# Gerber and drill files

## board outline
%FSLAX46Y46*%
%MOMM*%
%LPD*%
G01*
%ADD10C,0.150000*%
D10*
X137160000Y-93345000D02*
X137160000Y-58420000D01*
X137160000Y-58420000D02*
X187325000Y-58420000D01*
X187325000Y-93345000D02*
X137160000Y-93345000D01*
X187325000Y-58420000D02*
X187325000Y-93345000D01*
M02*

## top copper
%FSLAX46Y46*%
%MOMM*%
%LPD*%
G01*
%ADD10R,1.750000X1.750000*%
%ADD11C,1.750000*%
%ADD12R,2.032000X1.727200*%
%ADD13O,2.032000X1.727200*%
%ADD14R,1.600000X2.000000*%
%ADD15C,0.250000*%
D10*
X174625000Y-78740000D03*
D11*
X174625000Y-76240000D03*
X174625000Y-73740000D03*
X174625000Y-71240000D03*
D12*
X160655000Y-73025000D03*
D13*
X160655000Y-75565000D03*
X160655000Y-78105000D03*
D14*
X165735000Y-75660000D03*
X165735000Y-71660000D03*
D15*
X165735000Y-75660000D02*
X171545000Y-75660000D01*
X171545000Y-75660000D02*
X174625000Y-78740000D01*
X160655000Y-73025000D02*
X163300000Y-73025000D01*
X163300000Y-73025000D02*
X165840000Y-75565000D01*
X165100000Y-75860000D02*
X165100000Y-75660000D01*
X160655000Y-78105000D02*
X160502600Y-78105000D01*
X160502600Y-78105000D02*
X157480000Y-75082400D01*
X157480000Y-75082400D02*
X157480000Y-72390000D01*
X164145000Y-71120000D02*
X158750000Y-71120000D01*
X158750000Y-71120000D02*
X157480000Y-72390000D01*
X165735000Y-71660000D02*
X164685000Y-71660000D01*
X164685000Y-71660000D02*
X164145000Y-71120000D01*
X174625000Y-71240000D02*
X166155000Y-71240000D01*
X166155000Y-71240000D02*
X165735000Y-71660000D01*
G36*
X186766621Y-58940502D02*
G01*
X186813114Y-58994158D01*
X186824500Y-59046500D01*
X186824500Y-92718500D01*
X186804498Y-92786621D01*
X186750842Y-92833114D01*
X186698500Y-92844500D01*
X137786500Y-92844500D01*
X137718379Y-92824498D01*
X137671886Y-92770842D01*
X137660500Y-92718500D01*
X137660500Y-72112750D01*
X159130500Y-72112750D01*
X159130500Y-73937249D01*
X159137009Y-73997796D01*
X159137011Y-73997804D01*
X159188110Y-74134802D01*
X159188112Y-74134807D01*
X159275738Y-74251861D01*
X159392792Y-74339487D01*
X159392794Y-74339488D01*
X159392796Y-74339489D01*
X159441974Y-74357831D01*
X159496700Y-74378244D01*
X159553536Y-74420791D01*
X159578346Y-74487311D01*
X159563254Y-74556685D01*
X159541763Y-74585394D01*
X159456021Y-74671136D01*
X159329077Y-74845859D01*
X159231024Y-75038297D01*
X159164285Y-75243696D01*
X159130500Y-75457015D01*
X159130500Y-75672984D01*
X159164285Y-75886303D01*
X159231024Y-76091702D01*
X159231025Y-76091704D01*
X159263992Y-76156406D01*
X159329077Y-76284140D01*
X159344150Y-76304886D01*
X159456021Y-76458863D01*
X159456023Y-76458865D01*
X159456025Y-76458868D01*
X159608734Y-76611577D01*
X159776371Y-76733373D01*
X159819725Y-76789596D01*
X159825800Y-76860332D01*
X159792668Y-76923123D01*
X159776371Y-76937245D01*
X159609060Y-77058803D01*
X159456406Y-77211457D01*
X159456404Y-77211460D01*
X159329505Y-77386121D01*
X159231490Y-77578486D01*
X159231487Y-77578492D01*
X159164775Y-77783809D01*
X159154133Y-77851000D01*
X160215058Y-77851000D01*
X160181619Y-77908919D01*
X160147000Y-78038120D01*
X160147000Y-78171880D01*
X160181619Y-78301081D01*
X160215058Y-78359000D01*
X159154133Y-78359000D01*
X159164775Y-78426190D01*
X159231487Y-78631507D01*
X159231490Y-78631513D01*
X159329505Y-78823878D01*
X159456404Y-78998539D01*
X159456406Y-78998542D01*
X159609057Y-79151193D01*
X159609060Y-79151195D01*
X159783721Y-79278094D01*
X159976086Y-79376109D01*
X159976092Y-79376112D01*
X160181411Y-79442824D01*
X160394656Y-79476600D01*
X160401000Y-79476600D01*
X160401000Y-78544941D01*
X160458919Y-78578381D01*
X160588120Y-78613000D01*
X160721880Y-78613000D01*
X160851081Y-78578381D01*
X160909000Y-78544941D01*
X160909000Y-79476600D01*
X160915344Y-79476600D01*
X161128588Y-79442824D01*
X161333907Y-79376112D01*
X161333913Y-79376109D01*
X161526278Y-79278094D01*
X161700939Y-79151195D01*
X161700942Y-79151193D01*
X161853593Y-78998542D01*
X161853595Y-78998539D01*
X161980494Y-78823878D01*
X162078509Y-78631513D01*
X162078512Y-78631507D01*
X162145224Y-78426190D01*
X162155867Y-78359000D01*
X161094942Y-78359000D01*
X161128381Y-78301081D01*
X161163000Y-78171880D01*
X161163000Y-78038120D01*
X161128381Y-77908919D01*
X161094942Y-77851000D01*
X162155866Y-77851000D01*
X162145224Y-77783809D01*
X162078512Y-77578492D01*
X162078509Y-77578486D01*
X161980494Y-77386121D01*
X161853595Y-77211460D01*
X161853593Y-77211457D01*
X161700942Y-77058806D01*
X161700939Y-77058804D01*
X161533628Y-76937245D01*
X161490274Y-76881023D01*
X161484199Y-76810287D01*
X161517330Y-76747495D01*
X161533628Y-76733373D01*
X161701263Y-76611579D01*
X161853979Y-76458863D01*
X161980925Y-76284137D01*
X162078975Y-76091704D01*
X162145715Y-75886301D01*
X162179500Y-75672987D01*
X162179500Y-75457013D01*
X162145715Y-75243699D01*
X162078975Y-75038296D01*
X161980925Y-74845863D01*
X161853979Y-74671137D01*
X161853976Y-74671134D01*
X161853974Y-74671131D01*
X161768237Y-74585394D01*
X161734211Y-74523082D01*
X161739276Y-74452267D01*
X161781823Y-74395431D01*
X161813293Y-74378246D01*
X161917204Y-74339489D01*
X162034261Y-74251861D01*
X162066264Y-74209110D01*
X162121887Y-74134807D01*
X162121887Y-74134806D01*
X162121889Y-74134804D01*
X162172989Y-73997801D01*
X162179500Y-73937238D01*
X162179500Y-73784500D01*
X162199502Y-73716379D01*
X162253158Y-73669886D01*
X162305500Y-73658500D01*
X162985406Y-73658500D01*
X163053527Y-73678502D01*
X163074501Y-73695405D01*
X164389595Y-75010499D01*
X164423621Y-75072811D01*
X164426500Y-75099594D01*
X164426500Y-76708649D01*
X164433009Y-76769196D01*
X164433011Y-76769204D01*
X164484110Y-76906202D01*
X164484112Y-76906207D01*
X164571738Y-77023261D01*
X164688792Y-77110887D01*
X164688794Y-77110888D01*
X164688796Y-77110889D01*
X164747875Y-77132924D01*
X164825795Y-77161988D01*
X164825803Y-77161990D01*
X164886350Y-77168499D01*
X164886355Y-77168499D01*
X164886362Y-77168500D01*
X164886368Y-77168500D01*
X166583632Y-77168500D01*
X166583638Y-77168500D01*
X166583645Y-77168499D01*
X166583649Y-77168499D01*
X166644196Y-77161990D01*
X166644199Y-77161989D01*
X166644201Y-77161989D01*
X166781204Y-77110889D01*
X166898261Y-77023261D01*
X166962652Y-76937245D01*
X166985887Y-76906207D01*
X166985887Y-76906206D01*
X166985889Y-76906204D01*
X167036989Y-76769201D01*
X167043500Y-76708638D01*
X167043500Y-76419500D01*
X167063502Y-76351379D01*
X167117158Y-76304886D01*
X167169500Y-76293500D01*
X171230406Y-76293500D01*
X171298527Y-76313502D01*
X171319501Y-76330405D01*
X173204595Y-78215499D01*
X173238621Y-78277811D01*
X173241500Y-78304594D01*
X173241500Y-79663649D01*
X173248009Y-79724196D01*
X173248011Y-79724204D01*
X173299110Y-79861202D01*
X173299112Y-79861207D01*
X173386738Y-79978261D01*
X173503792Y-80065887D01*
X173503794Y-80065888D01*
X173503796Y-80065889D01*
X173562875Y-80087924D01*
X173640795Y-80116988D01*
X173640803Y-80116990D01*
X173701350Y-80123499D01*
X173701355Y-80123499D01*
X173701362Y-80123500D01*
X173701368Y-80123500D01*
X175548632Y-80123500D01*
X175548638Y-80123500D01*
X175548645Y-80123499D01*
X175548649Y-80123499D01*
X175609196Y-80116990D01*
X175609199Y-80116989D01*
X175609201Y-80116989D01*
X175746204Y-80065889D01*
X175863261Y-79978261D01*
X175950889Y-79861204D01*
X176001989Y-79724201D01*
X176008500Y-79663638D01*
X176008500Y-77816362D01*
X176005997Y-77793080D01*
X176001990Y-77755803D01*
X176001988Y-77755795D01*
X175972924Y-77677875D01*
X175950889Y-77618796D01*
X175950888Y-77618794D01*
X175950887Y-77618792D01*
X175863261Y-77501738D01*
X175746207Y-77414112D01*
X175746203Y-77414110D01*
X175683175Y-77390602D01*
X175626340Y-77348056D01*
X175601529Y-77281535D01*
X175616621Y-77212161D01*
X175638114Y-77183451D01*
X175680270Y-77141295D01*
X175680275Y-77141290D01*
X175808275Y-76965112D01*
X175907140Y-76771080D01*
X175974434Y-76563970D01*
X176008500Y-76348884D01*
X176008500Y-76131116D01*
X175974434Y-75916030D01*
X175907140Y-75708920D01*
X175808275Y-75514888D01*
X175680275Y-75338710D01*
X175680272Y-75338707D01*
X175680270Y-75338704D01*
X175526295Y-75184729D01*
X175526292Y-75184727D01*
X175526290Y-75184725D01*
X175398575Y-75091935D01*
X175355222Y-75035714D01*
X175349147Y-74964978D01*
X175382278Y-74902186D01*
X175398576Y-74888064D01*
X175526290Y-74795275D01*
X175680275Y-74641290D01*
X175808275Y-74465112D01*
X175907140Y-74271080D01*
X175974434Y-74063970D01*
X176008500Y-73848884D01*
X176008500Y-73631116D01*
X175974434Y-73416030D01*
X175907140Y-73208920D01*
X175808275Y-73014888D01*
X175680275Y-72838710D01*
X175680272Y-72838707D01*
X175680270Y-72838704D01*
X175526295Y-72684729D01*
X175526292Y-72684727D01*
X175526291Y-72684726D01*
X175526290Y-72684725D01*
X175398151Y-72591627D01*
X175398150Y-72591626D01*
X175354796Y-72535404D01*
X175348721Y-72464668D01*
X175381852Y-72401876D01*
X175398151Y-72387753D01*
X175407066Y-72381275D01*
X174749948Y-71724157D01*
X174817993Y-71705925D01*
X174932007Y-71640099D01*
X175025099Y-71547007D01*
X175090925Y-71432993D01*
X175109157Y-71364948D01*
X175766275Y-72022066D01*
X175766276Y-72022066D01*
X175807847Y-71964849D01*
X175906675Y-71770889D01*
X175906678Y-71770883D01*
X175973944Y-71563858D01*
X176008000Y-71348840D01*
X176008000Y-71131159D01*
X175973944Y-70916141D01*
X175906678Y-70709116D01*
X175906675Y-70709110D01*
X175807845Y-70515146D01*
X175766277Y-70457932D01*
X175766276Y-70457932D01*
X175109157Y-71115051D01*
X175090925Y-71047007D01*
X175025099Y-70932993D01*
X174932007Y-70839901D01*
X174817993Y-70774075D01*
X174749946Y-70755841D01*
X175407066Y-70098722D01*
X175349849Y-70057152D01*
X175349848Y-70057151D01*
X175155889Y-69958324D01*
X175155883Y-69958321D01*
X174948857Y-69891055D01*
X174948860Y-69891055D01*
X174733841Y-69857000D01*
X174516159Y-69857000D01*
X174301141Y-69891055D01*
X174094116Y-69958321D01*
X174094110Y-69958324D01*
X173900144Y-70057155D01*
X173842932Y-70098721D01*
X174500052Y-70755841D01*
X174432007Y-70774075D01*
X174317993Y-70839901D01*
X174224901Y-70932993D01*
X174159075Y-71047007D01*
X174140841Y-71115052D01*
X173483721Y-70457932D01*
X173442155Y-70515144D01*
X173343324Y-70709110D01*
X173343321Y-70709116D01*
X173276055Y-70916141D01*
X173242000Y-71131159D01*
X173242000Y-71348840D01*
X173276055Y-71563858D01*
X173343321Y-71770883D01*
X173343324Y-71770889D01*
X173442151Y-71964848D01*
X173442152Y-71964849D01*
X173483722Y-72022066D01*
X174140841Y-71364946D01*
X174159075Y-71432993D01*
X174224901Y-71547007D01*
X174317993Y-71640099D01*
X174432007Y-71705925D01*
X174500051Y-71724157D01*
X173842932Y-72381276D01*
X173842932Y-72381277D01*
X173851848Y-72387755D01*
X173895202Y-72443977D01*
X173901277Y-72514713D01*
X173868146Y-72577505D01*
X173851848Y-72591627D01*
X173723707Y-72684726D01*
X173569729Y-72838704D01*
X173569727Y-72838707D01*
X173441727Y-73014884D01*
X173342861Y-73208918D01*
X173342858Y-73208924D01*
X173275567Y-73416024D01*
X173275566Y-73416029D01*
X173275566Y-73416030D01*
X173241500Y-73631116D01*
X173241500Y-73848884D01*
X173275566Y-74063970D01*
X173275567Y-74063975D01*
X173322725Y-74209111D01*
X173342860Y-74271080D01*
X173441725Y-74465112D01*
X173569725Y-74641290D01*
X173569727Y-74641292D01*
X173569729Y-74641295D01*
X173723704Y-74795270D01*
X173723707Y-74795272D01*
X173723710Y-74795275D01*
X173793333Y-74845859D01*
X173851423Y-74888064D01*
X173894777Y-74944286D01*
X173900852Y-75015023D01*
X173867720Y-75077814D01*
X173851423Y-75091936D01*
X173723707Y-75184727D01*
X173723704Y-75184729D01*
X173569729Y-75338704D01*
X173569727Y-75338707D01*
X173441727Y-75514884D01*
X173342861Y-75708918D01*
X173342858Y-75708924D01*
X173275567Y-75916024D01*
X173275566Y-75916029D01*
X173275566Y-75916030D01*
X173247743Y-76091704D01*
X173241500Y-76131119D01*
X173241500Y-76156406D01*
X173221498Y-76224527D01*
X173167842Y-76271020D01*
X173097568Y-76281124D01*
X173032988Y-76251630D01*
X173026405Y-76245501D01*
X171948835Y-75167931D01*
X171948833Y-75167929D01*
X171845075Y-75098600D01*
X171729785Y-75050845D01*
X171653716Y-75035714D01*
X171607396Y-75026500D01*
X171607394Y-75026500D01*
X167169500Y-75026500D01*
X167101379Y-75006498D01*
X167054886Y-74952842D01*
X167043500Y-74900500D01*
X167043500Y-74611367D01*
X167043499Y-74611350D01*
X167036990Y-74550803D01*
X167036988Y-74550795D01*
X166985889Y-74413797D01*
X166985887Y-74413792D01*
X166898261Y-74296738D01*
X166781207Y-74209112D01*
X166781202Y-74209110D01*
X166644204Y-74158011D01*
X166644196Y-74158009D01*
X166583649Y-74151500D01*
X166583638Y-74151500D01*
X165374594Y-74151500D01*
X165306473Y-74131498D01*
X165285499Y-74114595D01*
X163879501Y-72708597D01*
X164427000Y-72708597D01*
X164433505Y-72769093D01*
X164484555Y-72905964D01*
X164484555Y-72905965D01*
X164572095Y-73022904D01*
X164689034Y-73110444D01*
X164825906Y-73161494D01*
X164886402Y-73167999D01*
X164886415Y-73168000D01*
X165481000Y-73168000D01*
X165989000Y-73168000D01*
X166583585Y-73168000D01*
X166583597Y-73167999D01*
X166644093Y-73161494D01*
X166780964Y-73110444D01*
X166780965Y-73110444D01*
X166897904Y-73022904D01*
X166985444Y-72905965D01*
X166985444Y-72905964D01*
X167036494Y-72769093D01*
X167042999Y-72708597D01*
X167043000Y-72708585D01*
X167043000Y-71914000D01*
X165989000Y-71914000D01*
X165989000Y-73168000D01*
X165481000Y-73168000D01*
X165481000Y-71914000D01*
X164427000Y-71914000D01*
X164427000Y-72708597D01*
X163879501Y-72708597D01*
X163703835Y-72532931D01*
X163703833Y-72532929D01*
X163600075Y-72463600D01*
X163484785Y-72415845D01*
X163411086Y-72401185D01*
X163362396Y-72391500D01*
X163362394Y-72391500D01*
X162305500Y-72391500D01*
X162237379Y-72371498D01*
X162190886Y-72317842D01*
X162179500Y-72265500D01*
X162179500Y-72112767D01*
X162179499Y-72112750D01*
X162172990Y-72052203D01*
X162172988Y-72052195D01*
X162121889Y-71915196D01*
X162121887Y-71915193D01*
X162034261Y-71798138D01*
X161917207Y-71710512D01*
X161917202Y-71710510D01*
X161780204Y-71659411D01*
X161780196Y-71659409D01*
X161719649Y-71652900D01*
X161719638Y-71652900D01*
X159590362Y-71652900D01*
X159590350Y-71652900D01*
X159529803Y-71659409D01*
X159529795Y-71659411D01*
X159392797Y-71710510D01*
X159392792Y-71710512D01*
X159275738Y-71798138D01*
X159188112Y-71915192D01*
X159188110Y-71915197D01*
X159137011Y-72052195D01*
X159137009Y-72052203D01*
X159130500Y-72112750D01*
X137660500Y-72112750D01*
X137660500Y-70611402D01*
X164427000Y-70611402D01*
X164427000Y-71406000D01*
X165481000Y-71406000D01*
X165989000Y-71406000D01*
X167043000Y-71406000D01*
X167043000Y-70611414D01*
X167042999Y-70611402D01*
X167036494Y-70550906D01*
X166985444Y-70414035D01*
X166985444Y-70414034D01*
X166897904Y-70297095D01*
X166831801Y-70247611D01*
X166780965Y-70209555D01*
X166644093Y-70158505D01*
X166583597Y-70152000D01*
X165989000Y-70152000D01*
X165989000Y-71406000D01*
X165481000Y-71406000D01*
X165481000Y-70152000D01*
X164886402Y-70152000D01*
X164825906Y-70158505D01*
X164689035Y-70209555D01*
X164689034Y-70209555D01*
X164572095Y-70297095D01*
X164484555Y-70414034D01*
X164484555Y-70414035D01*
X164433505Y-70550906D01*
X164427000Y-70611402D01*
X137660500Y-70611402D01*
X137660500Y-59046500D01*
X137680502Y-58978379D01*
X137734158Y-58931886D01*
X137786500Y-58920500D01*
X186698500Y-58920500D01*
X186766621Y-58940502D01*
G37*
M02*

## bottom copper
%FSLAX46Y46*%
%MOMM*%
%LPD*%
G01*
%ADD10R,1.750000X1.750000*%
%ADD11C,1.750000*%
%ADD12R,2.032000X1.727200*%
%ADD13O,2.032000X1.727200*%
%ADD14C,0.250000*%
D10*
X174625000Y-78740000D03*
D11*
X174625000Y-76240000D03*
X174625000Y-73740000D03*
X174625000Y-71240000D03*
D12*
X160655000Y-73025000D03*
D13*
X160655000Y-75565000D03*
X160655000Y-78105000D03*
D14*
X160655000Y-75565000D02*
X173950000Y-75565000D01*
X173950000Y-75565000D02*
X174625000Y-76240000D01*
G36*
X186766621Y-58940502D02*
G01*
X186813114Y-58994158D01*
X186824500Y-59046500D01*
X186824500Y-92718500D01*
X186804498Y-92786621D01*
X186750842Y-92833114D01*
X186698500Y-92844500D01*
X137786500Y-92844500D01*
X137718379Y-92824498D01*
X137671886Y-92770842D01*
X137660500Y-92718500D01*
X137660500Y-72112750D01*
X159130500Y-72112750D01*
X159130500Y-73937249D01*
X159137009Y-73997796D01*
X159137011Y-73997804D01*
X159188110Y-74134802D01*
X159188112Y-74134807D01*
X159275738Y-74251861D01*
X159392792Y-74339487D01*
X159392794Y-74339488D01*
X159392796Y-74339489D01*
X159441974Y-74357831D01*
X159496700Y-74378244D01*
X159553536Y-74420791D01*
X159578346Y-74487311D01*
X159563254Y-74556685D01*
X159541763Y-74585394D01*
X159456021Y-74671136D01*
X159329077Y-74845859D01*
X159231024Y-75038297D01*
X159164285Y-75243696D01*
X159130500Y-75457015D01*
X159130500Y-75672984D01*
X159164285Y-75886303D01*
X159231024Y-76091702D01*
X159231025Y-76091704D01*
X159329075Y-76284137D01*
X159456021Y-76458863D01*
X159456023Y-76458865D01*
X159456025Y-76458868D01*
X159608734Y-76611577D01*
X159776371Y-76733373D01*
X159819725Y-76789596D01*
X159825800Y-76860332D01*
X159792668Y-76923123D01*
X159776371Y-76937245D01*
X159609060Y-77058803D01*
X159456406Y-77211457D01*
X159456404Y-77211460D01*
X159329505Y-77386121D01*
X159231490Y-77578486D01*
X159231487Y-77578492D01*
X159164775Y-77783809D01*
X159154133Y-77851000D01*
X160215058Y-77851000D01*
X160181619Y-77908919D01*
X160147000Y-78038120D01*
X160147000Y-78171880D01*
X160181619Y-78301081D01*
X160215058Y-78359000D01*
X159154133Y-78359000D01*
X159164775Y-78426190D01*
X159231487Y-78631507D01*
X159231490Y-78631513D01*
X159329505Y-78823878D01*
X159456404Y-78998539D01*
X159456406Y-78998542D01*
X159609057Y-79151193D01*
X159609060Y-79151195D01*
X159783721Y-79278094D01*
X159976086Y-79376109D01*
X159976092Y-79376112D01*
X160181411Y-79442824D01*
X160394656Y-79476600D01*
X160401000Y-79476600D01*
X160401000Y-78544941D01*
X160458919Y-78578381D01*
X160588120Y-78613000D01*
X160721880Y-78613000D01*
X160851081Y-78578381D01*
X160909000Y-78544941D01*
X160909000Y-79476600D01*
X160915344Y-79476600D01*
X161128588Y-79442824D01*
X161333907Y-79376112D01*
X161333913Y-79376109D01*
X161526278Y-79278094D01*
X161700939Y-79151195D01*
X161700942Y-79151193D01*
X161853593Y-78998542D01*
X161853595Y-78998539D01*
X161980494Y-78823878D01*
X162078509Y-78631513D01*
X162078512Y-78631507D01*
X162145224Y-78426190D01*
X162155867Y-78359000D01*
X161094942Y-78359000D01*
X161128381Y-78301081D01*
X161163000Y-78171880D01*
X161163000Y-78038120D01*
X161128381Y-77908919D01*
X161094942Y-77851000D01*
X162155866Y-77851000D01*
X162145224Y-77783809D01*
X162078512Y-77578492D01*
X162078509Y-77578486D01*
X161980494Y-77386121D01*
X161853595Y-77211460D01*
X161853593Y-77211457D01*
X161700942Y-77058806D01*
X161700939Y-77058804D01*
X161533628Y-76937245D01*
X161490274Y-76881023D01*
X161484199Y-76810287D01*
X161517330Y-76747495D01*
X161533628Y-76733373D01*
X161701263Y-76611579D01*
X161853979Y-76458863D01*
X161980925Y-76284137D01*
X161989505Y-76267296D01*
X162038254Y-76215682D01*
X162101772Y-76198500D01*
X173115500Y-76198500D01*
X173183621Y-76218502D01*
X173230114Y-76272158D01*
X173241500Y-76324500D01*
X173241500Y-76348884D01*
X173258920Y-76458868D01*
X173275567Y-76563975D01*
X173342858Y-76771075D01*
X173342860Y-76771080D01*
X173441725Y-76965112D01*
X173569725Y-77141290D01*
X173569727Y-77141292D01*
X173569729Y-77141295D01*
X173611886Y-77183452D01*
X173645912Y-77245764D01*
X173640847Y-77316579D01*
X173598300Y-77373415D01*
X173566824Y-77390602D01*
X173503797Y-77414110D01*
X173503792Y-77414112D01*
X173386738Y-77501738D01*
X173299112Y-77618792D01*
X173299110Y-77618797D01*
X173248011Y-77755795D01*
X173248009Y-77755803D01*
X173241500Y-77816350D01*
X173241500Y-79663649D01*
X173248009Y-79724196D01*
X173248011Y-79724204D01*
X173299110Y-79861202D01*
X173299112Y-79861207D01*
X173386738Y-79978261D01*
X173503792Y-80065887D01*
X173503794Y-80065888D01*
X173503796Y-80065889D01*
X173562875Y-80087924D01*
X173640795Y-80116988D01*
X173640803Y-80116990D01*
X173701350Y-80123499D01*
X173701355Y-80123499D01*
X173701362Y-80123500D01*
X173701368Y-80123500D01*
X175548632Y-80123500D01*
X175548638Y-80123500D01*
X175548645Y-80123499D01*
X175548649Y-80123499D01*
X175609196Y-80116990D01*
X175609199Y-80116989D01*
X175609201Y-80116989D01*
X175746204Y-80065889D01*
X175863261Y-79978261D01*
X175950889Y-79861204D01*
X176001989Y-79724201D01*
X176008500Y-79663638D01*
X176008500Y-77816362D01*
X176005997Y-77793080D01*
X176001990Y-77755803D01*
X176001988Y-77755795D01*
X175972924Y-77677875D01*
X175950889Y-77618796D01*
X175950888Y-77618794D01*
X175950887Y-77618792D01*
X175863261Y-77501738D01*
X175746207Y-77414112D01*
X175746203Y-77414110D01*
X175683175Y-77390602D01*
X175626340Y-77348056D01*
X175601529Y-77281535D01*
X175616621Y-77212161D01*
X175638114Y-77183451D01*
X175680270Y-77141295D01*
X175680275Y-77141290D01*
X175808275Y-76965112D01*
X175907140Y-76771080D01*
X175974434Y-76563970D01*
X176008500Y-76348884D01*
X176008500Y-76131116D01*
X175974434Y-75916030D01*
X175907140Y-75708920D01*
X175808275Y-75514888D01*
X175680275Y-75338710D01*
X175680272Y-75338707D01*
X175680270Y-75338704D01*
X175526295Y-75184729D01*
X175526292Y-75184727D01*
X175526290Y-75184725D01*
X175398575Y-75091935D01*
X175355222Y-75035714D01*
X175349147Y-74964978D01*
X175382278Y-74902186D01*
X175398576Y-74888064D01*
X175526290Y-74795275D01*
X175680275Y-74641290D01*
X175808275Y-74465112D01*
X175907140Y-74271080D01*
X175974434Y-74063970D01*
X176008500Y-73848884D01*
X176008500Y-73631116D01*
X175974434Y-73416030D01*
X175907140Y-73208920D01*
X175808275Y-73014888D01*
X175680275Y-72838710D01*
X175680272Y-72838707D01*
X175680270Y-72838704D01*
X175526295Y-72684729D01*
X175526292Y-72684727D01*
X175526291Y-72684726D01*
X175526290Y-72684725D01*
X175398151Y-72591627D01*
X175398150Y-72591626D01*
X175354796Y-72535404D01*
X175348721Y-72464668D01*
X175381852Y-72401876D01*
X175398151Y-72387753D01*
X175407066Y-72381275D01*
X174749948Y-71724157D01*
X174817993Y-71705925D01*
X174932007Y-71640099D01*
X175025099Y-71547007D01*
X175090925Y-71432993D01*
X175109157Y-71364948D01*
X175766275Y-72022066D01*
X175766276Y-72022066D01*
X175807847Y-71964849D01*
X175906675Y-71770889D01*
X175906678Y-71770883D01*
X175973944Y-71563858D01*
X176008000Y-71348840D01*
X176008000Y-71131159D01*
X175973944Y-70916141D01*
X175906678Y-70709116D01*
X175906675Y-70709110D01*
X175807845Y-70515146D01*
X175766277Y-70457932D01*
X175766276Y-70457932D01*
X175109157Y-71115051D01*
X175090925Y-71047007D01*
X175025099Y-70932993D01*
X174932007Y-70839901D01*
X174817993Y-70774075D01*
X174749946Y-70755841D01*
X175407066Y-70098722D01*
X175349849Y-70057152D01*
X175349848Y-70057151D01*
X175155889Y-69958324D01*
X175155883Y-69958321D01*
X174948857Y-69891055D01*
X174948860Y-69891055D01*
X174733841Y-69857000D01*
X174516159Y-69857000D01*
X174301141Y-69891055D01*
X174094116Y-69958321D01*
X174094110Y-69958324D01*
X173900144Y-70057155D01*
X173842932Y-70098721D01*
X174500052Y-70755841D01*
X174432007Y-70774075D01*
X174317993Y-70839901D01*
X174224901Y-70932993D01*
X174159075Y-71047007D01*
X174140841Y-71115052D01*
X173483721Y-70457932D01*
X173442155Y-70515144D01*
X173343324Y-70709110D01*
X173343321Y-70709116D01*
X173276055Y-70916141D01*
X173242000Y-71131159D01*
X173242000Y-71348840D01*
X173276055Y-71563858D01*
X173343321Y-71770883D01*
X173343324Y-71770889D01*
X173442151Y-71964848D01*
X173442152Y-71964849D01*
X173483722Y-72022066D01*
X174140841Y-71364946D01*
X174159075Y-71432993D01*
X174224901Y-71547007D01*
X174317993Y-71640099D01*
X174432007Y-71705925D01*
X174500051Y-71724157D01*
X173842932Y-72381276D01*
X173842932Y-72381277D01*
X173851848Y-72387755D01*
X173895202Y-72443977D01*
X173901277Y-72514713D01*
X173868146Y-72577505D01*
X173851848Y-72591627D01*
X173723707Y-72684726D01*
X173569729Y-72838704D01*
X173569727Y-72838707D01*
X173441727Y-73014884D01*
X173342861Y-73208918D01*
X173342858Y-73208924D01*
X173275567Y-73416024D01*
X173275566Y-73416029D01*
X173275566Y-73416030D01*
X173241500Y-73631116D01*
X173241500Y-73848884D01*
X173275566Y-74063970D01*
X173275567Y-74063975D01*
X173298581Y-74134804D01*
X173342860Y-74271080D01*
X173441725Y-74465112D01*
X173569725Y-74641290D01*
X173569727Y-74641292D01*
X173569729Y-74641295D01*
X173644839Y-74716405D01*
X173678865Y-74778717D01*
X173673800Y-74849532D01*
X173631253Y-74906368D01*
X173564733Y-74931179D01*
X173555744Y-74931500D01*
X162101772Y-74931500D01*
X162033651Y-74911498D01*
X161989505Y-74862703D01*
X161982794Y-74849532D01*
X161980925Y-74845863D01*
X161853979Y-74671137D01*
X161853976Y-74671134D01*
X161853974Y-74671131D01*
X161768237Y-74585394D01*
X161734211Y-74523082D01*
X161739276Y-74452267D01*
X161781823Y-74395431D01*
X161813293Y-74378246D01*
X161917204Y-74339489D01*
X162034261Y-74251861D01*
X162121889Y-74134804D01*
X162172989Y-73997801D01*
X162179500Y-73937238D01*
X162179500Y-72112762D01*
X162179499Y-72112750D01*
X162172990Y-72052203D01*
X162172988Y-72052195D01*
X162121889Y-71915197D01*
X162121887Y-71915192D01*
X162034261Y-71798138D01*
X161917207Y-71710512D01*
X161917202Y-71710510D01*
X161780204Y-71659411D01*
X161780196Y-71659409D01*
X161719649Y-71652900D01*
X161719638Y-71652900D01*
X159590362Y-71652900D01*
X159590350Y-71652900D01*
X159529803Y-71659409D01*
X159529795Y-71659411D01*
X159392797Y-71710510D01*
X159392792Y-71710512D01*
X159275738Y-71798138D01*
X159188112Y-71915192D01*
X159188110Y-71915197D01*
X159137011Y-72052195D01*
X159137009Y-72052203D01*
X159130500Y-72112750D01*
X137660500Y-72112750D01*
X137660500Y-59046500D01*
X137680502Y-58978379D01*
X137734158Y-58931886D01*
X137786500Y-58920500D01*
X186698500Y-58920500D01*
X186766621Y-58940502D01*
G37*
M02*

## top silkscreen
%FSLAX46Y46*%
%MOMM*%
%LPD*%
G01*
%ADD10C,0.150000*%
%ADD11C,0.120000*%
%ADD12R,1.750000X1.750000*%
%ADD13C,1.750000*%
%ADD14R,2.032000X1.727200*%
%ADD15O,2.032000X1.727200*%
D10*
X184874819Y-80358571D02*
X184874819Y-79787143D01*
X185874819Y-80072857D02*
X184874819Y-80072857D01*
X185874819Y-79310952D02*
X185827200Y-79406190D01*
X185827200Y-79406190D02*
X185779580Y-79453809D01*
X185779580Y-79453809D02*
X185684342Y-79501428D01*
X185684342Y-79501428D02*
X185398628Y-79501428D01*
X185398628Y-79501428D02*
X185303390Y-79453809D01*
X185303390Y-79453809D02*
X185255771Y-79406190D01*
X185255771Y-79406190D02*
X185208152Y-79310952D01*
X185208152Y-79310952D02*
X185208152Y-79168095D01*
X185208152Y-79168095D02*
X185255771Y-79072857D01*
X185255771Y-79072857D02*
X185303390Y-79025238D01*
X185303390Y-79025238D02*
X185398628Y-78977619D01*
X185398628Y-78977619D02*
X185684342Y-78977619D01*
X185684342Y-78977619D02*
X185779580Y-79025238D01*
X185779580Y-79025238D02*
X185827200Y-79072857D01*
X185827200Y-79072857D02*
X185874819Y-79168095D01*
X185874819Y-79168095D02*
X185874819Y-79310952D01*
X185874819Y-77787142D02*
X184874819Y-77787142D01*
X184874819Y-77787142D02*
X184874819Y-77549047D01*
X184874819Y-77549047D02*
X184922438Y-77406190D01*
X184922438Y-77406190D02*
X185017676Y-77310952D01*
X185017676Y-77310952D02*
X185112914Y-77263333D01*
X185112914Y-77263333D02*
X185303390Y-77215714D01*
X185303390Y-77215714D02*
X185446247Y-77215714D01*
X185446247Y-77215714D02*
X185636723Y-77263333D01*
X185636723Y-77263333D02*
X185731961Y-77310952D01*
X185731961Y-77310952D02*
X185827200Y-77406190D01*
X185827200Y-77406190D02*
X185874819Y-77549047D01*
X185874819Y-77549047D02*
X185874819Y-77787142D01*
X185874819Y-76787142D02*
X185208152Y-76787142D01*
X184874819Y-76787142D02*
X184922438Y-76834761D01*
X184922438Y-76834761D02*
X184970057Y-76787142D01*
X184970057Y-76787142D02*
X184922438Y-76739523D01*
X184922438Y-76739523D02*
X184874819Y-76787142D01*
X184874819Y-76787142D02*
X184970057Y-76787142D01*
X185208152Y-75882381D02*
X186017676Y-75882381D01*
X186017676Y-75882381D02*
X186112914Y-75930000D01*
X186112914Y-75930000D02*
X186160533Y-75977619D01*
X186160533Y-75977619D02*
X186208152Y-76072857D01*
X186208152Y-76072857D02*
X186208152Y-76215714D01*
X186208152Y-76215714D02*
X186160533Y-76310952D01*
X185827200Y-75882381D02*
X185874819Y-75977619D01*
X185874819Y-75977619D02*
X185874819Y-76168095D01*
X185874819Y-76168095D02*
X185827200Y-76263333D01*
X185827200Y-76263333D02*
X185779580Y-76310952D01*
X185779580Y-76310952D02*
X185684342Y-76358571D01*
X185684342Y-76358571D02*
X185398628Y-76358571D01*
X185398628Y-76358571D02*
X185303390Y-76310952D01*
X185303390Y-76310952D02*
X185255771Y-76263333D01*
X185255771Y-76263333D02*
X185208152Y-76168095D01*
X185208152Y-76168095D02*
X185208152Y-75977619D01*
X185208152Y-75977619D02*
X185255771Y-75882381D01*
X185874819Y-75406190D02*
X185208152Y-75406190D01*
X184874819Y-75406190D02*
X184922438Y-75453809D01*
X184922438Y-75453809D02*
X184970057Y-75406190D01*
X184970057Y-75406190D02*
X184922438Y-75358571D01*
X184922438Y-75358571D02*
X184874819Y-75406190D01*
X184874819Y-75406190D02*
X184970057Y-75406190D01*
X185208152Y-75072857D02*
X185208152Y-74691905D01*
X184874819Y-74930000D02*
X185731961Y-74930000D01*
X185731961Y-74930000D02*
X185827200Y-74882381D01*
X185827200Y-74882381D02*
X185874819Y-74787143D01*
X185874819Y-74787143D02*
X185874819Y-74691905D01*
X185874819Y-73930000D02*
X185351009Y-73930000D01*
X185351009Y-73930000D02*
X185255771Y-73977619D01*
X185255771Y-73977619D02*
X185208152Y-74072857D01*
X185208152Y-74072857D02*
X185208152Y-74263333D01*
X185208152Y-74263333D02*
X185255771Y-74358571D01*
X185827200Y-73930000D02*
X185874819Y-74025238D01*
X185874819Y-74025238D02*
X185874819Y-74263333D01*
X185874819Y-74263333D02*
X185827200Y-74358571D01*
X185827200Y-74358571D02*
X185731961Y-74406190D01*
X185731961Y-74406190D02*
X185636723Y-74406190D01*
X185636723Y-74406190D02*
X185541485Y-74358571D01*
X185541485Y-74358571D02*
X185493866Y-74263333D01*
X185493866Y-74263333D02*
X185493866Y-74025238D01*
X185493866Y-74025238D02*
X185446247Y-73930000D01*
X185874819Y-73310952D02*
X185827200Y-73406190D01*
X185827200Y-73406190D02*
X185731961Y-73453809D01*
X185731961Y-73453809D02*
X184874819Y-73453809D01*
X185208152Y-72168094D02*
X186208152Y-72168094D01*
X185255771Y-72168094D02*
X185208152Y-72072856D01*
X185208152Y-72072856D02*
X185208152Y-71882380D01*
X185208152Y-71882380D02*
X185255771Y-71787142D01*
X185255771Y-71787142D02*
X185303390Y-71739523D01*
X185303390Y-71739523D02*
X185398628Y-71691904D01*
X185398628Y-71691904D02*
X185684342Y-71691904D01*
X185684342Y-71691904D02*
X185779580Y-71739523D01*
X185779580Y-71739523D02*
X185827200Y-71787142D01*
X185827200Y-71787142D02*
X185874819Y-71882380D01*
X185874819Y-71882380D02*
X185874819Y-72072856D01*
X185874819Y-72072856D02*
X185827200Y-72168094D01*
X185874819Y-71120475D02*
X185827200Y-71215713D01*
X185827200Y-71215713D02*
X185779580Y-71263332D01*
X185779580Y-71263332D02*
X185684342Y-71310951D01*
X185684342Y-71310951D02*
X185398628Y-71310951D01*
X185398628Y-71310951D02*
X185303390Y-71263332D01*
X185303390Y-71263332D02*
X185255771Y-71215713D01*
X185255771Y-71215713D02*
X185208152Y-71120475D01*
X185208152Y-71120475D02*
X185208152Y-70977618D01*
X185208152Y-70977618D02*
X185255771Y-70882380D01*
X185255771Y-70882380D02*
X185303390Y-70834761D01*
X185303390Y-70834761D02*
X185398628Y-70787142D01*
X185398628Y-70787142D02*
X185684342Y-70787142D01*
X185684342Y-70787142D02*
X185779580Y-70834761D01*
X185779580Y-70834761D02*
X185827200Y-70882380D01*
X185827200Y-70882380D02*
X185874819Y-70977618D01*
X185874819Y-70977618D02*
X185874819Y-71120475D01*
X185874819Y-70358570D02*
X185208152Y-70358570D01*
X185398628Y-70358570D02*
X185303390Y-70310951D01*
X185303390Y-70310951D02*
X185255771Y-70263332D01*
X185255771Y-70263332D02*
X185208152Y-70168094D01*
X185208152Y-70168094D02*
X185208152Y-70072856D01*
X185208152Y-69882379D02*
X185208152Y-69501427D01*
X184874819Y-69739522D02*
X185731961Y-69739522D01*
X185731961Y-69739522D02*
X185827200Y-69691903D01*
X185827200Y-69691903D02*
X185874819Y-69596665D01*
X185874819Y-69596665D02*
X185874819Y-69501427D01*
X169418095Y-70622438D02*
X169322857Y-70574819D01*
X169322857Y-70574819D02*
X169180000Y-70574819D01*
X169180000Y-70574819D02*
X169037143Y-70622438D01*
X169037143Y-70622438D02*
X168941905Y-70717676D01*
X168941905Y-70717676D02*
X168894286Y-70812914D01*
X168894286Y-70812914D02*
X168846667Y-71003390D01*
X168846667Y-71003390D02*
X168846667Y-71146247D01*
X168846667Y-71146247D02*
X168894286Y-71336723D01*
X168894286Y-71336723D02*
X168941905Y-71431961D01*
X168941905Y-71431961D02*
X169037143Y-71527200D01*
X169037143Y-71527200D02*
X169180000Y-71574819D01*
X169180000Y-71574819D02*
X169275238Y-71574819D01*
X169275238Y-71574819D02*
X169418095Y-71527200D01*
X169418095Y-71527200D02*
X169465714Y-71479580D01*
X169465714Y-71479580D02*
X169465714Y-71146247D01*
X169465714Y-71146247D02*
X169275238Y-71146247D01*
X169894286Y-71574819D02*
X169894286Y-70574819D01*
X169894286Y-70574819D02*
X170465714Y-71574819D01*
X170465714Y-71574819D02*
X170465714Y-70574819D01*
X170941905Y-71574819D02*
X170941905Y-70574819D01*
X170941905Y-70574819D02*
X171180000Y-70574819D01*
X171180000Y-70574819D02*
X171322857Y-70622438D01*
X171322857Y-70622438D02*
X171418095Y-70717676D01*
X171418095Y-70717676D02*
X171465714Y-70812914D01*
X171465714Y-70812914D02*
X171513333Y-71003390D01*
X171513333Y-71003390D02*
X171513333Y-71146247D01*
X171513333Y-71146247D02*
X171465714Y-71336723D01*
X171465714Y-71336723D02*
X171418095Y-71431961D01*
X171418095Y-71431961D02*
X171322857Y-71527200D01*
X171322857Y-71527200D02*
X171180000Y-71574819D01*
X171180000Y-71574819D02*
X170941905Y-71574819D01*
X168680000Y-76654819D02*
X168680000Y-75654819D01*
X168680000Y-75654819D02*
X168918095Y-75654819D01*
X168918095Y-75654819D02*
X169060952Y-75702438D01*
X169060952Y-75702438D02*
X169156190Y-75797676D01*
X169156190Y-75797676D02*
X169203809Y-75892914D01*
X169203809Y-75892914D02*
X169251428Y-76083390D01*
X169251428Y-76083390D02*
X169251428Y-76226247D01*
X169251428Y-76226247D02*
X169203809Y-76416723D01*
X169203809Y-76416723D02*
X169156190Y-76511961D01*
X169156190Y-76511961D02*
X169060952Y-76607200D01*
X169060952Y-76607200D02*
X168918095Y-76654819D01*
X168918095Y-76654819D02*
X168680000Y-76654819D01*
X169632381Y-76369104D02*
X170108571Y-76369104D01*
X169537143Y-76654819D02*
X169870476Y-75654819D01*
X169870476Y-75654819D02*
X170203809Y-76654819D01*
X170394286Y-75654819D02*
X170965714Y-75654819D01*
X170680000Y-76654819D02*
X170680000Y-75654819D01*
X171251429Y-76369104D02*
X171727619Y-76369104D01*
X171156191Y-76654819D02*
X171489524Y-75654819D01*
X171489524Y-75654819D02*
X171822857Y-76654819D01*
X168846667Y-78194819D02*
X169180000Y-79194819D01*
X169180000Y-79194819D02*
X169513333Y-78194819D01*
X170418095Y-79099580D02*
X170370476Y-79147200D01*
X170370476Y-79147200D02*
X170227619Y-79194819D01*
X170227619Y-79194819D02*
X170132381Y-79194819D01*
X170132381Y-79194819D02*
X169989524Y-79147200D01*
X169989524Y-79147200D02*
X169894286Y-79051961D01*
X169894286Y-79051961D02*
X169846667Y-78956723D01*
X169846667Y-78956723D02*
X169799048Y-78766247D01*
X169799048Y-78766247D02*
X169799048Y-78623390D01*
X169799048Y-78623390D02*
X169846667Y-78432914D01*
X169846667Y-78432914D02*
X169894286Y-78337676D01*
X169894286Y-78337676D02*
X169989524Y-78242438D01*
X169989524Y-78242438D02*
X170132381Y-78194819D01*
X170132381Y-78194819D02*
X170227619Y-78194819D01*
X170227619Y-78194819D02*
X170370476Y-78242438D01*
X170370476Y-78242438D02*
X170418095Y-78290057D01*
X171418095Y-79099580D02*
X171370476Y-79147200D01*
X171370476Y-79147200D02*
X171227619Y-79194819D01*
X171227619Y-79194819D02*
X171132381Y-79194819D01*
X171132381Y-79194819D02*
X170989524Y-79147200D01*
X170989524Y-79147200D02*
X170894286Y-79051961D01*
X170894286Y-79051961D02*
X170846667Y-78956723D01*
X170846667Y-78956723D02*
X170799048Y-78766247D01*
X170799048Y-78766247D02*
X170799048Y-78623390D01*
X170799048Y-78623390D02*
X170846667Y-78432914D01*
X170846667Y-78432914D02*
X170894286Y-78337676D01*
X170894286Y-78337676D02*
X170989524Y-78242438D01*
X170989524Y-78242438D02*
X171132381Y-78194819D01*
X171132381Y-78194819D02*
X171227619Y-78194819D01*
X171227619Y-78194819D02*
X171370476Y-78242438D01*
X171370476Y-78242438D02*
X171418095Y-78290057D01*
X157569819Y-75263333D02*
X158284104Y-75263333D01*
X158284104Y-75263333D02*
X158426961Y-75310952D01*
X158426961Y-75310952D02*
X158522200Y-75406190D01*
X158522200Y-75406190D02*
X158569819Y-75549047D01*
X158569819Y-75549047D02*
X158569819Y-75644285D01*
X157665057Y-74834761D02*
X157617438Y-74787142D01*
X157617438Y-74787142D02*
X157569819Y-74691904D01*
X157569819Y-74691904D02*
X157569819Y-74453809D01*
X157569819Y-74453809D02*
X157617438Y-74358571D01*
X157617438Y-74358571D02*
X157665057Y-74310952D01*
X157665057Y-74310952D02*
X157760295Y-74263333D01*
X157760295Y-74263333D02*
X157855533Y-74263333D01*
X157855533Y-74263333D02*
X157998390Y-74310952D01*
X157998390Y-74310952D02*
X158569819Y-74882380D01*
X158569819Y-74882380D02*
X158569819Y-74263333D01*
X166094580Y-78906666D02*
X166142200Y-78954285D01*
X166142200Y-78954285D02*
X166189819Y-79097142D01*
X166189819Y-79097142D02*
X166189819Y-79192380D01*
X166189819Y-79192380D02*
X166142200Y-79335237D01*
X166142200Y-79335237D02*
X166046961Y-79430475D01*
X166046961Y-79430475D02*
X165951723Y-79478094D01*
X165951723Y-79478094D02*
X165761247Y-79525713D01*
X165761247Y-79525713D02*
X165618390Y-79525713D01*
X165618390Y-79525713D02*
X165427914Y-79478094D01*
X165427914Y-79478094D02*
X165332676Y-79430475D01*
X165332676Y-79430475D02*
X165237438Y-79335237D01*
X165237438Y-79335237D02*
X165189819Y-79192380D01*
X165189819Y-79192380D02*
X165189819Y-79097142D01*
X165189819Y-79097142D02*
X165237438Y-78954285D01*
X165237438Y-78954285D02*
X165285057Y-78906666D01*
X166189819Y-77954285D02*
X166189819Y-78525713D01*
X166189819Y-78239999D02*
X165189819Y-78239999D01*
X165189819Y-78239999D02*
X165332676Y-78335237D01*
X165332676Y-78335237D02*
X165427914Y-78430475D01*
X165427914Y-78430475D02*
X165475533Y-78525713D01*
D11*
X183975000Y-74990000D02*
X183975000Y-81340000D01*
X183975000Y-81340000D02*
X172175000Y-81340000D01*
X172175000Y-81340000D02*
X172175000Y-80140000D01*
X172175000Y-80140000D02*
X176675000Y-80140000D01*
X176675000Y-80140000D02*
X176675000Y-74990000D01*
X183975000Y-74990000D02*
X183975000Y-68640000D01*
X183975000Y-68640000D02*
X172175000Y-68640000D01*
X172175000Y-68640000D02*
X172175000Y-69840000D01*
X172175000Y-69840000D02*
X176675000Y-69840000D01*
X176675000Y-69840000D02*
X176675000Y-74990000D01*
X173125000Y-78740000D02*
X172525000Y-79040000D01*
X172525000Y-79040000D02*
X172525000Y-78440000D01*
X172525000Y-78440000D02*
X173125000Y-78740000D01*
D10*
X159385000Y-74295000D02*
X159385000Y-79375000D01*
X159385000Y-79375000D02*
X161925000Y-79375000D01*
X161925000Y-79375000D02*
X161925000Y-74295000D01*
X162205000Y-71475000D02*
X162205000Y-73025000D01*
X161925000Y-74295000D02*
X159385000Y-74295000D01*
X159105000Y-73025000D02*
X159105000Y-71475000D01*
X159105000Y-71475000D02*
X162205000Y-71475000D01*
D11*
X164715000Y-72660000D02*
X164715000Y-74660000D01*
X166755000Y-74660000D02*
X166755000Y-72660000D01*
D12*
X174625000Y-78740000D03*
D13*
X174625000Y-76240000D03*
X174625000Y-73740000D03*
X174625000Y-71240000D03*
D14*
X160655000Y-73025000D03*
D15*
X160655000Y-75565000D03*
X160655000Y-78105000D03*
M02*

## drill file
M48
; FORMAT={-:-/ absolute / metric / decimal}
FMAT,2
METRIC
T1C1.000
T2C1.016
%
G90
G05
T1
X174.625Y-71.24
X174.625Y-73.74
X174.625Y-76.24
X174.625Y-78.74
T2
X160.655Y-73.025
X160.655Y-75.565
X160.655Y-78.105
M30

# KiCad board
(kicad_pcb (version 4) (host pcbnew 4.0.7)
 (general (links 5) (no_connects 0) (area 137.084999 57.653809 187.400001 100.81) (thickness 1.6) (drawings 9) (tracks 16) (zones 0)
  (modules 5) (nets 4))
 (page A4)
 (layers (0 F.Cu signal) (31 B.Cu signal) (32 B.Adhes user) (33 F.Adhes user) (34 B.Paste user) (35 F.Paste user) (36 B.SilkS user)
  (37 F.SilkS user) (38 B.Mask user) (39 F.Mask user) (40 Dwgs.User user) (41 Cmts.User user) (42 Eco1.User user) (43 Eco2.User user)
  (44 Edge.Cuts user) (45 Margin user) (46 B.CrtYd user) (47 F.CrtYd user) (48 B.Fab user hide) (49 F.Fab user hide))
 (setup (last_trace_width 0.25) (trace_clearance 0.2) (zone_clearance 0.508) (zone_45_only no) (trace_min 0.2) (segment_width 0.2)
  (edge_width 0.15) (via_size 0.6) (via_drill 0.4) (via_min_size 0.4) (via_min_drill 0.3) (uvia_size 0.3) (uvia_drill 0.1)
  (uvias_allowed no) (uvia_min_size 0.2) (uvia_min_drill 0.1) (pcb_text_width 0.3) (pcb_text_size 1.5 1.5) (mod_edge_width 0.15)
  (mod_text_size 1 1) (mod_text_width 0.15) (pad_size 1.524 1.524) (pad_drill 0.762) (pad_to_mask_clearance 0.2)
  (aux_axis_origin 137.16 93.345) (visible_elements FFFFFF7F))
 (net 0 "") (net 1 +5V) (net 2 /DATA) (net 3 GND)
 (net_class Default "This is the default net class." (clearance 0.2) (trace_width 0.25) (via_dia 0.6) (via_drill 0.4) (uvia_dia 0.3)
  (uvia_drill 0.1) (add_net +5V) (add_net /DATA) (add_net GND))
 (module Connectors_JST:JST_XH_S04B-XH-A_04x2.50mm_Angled (layer F.Cu) (at 174.625 78.74 90)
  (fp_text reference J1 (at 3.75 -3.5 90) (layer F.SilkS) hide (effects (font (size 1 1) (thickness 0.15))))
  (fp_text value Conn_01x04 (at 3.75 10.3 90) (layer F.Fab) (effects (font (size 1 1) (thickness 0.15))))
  (fp_line (start 3.75 9.35) (end -2.6 9.35) (layer F.SilkS) (width 0.12))
  (fp_line (start -2.6 9.35) (end -2.6 -2.45) (layer F.SilkS) (width 0.12))
  (fp_line (start -2.6 -2.45) (end -1.4 -2.45) (layer F.SilkS) (width 0.12))
  (fp_line (start -1.4 -2.45) (end -1.4 2.05) (layer F.SilkS) (width 0.12))
  (fp_line (start -1.4 2.05) (end 3.75 2.05) (layer F.SilkS) (width 0.12))
  (fp_line (start 3.75 9.35) (end 10.1 9.35) (layer F.SilkS) (width 0.12))
  (fp_line (start 10.1 9.35) (end 10.1 -2.45) (layer F.SilkS) (width 0.12))
  (fp_line (start 10.1 -2.45) (end 8.9 -2.45) (layer F.SilkS) (width 0.12))
  (fp_line (start 8.9 -2.45) (end 8.9 2.05) (layer F.SilkS) (width 0.12))
  (fp_line (start 8.9 2.05) (end 3.75 2.05) (layer F.SilkS) (width 0.12))
  (fp_line (start 0 -1.5) (end -0.3 -2.1) (layer F.SilkS) (width 0.12))
  (fp_line (start -0.3 -2.1) (end 0.3 -2.1) (layer F.SilkS) (width 0.12))
  (fp_line (start 0.3 -2.1) (end 0 -1.5) (layer F.SilkS) (width 0.12))
  (pad 1 thru_hole rect (at 0 0 90) (size 1.75 1.75) (drill 1) (layers *.Cu *.Mask F.SilkS) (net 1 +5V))
  (pad 2 thru_hole circle (at 2.5 0 90) (size 1.75 1.75) (drill 1) (layers *.Cu *.Mask F.SilkS) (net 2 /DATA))
  (pad 3 thru_hole circle (at 5 0 90) (size 1.75 1.75) (drill 1) (layers *.Cu *.Mask F.SilkS))
  (pad 4 thru_hole circle (at 7.5 0 90) (size 1.75 1.75) (drill 1) (layers *.Cu *.Mask F.SilkS) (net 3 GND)))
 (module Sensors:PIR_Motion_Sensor (layer F.Cu) (at 160.655 75.565 270)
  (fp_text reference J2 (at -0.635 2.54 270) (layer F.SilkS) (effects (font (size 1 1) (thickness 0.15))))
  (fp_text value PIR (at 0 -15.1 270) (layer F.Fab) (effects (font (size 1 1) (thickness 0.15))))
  (fp_line (start -1.27 1.27) (end 3.81 1.27) (layer F.SilkS) (width 0.15))
  (fp_line (start 3.81 1.27) (end 3.81 -1.27) (layer F.SilkS) (width 0.15))
  (fp_line (start 3.81 -1.27) (end -1.27 -1.27) (layer F.SilkS) (width 0.15))
  (fp_line (start -4.09 -1.55) (end -2.54 -1.55) (layer F.SilkS) (width 0.15))
  (fp_line (start -1.27 -1.27) (end -1.27 1.27) (layer F.SilkS) (width 0.15))
  (fp_line (start -2.54 1.55) (end -4.09 1.55) (layer F.SilkS) (width 0.15))
  (fp_line (start -4.09 1.55) (end -4.09 -1.55) (layer F.SilkS) (width 0.15))
  (pad 1 thru_hole rect (at -2.54 0) (size 2.032 1.7272) (drill 1.016) (layers *.Cu *.Mask F.SilkS) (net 1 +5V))
  (pad 2 thru_hole oval (at 0 0) (size 2.032 1.7272) (drill 1.016) (layers *.Cu *.Mask F.SilkS) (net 2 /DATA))
  (pad 3 thru_hole oval (at 2.54 0) (size 2.032 1.7272) (drill 1.016) (layers *.Cu *.Mask F.SilkS) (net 3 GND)))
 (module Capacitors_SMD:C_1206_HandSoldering (layer F.Cu) (at 165.735 73.66 90)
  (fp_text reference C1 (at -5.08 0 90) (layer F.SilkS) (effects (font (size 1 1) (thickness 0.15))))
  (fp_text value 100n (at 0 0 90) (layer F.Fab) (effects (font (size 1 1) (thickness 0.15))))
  (fp_line (start 1 -1.02) (end -1 -1.02) (layer F.SilkS) (width 0.12))
  (fp_line (start -1 1.02) (end 1 1.02) (layer F.SilkS) (width 0.12))
  (pad 1 smd rect (at -2 0 90) (size 2 1.6) (layers F.Cu F.Paste F.Mask) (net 1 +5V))
  (pad 2 smd rect (at 2 0 90) (size 2 1.6) (layers F.Cu F.Paste F.Mask) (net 3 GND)))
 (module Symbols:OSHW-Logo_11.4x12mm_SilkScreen (layer B.Cu) (at 167.005 86.36 270)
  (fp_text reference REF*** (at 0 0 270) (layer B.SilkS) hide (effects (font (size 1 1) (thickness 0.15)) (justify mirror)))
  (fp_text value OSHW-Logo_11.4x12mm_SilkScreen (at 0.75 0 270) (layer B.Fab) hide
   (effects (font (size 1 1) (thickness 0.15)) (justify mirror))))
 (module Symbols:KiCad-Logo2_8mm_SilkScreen (layer B.Cu) (at 167.64 68.58 270)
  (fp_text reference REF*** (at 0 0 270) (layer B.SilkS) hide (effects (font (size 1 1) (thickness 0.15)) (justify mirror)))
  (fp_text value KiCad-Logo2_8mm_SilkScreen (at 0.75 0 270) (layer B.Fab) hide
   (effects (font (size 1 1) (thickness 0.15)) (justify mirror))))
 (gr_line (start 137.16 93.345) (end 137.16 58.42) (layer Edge.Cuts) (width 0.15))
 (gr_line (start 137.16 58.42) (end 187.325 58.42) (layer Edge.Cuts) (width 0.15))
 (gr_line (start 187.325 93.345) (end 137.16 93.345) (layer Edge.Cuts) (width 0.15))
 (gr_line (start 187.325 58.42) (end 187.325 93.345) (layer Edge.Cuts) (width 0.15))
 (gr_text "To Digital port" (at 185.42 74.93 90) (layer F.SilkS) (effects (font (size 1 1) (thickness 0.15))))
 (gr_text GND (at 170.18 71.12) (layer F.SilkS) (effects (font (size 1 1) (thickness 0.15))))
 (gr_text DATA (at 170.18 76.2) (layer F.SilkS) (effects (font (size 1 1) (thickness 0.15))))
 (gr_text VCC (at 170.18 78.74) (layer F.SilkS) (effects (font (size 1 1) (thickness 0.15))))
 (segment (start 165.735 75.66) (end 171.545 75.66) (width 0.25) (layer F.Cu) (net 1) (status 10))
 (segment (start 171.545 75.66) (end 174.625 78.74) (width 0.25) (layer F.Cu) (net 1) (status 20))
 (segment (start 160.655 73.025) (end 163.3 73.025) (width 0.25) (layer F.Cu) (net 1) (status 10))
 (segment (start 163.3 73.025) (end 165.84 75.565) (width 0.25) (layer F.Cu) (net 1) (status 20))
 (segment (start 165.1 75.86) (end 165.1 75.66) (width 0.25) (layer F.Cu) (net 1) (status 30))
 (segment (start 160.655 78.105) (end 160.5026 78.105) (width 0.25) (layer F.Cu) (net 3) (status 30))
 (segment (start 160.5026 78.105) (end 157.48 75.0824) (width 0.25) (layer F.Cu) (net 3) (status 10))
 (segment (start 157.48 75.0824) (end 157.48 72.39) (width 0.25) (layer F.Cu) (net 3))
 (segment (start 164.145 71.12) (end 158.75 71.12) (width 0.25) (layer F.Cu) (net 3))
 (segment (start 158.75 71.12) (end 157.48 72.39) (width 0.25) (layer F.Cu) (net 3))
 (segment (start 165.735 71.66) (end 164.685 71.66) (width 0.25) (layer F.Cu) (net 3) (status 10))
 (segment (start 164.685 71.66) (end 164.145 71.12) (width 0.25) (layer F.Cu) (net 3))
 (segment (start 174.625 71.24) (end 166.155 71.24) (width 0.25) (layer F.Cu) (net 3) (status 30))
 (segment (start 166.155 71.24) (end 165.735 71.66) (width 0.25) (layer F.Cu) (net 3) (status 30))
 (segment (start 160.655 75.565) (end 173.95 75.565) (width 0.25) (layer B.Cu) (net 2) (status 10))
 (segment (start 173.95 75.565) (end 174.625 76.24) (width 0.25) (layer B.Cu) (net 2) (status 20))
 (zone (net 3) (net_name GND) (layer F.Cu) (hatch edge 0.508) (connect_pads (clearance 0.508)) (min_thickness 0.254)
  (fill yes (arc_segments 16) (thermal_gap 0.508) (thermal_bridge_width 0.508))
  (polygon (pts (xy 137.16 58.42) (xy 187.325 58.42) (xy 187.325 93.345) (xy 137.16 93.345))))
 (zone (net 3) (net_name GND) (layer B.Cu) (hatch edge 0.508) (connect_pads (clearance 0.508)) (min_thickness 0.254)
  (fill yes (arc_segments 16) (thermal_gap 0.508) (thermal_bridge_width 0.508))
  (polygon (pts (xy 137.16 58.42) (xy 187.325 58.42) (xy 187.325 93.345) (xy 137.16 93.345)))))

